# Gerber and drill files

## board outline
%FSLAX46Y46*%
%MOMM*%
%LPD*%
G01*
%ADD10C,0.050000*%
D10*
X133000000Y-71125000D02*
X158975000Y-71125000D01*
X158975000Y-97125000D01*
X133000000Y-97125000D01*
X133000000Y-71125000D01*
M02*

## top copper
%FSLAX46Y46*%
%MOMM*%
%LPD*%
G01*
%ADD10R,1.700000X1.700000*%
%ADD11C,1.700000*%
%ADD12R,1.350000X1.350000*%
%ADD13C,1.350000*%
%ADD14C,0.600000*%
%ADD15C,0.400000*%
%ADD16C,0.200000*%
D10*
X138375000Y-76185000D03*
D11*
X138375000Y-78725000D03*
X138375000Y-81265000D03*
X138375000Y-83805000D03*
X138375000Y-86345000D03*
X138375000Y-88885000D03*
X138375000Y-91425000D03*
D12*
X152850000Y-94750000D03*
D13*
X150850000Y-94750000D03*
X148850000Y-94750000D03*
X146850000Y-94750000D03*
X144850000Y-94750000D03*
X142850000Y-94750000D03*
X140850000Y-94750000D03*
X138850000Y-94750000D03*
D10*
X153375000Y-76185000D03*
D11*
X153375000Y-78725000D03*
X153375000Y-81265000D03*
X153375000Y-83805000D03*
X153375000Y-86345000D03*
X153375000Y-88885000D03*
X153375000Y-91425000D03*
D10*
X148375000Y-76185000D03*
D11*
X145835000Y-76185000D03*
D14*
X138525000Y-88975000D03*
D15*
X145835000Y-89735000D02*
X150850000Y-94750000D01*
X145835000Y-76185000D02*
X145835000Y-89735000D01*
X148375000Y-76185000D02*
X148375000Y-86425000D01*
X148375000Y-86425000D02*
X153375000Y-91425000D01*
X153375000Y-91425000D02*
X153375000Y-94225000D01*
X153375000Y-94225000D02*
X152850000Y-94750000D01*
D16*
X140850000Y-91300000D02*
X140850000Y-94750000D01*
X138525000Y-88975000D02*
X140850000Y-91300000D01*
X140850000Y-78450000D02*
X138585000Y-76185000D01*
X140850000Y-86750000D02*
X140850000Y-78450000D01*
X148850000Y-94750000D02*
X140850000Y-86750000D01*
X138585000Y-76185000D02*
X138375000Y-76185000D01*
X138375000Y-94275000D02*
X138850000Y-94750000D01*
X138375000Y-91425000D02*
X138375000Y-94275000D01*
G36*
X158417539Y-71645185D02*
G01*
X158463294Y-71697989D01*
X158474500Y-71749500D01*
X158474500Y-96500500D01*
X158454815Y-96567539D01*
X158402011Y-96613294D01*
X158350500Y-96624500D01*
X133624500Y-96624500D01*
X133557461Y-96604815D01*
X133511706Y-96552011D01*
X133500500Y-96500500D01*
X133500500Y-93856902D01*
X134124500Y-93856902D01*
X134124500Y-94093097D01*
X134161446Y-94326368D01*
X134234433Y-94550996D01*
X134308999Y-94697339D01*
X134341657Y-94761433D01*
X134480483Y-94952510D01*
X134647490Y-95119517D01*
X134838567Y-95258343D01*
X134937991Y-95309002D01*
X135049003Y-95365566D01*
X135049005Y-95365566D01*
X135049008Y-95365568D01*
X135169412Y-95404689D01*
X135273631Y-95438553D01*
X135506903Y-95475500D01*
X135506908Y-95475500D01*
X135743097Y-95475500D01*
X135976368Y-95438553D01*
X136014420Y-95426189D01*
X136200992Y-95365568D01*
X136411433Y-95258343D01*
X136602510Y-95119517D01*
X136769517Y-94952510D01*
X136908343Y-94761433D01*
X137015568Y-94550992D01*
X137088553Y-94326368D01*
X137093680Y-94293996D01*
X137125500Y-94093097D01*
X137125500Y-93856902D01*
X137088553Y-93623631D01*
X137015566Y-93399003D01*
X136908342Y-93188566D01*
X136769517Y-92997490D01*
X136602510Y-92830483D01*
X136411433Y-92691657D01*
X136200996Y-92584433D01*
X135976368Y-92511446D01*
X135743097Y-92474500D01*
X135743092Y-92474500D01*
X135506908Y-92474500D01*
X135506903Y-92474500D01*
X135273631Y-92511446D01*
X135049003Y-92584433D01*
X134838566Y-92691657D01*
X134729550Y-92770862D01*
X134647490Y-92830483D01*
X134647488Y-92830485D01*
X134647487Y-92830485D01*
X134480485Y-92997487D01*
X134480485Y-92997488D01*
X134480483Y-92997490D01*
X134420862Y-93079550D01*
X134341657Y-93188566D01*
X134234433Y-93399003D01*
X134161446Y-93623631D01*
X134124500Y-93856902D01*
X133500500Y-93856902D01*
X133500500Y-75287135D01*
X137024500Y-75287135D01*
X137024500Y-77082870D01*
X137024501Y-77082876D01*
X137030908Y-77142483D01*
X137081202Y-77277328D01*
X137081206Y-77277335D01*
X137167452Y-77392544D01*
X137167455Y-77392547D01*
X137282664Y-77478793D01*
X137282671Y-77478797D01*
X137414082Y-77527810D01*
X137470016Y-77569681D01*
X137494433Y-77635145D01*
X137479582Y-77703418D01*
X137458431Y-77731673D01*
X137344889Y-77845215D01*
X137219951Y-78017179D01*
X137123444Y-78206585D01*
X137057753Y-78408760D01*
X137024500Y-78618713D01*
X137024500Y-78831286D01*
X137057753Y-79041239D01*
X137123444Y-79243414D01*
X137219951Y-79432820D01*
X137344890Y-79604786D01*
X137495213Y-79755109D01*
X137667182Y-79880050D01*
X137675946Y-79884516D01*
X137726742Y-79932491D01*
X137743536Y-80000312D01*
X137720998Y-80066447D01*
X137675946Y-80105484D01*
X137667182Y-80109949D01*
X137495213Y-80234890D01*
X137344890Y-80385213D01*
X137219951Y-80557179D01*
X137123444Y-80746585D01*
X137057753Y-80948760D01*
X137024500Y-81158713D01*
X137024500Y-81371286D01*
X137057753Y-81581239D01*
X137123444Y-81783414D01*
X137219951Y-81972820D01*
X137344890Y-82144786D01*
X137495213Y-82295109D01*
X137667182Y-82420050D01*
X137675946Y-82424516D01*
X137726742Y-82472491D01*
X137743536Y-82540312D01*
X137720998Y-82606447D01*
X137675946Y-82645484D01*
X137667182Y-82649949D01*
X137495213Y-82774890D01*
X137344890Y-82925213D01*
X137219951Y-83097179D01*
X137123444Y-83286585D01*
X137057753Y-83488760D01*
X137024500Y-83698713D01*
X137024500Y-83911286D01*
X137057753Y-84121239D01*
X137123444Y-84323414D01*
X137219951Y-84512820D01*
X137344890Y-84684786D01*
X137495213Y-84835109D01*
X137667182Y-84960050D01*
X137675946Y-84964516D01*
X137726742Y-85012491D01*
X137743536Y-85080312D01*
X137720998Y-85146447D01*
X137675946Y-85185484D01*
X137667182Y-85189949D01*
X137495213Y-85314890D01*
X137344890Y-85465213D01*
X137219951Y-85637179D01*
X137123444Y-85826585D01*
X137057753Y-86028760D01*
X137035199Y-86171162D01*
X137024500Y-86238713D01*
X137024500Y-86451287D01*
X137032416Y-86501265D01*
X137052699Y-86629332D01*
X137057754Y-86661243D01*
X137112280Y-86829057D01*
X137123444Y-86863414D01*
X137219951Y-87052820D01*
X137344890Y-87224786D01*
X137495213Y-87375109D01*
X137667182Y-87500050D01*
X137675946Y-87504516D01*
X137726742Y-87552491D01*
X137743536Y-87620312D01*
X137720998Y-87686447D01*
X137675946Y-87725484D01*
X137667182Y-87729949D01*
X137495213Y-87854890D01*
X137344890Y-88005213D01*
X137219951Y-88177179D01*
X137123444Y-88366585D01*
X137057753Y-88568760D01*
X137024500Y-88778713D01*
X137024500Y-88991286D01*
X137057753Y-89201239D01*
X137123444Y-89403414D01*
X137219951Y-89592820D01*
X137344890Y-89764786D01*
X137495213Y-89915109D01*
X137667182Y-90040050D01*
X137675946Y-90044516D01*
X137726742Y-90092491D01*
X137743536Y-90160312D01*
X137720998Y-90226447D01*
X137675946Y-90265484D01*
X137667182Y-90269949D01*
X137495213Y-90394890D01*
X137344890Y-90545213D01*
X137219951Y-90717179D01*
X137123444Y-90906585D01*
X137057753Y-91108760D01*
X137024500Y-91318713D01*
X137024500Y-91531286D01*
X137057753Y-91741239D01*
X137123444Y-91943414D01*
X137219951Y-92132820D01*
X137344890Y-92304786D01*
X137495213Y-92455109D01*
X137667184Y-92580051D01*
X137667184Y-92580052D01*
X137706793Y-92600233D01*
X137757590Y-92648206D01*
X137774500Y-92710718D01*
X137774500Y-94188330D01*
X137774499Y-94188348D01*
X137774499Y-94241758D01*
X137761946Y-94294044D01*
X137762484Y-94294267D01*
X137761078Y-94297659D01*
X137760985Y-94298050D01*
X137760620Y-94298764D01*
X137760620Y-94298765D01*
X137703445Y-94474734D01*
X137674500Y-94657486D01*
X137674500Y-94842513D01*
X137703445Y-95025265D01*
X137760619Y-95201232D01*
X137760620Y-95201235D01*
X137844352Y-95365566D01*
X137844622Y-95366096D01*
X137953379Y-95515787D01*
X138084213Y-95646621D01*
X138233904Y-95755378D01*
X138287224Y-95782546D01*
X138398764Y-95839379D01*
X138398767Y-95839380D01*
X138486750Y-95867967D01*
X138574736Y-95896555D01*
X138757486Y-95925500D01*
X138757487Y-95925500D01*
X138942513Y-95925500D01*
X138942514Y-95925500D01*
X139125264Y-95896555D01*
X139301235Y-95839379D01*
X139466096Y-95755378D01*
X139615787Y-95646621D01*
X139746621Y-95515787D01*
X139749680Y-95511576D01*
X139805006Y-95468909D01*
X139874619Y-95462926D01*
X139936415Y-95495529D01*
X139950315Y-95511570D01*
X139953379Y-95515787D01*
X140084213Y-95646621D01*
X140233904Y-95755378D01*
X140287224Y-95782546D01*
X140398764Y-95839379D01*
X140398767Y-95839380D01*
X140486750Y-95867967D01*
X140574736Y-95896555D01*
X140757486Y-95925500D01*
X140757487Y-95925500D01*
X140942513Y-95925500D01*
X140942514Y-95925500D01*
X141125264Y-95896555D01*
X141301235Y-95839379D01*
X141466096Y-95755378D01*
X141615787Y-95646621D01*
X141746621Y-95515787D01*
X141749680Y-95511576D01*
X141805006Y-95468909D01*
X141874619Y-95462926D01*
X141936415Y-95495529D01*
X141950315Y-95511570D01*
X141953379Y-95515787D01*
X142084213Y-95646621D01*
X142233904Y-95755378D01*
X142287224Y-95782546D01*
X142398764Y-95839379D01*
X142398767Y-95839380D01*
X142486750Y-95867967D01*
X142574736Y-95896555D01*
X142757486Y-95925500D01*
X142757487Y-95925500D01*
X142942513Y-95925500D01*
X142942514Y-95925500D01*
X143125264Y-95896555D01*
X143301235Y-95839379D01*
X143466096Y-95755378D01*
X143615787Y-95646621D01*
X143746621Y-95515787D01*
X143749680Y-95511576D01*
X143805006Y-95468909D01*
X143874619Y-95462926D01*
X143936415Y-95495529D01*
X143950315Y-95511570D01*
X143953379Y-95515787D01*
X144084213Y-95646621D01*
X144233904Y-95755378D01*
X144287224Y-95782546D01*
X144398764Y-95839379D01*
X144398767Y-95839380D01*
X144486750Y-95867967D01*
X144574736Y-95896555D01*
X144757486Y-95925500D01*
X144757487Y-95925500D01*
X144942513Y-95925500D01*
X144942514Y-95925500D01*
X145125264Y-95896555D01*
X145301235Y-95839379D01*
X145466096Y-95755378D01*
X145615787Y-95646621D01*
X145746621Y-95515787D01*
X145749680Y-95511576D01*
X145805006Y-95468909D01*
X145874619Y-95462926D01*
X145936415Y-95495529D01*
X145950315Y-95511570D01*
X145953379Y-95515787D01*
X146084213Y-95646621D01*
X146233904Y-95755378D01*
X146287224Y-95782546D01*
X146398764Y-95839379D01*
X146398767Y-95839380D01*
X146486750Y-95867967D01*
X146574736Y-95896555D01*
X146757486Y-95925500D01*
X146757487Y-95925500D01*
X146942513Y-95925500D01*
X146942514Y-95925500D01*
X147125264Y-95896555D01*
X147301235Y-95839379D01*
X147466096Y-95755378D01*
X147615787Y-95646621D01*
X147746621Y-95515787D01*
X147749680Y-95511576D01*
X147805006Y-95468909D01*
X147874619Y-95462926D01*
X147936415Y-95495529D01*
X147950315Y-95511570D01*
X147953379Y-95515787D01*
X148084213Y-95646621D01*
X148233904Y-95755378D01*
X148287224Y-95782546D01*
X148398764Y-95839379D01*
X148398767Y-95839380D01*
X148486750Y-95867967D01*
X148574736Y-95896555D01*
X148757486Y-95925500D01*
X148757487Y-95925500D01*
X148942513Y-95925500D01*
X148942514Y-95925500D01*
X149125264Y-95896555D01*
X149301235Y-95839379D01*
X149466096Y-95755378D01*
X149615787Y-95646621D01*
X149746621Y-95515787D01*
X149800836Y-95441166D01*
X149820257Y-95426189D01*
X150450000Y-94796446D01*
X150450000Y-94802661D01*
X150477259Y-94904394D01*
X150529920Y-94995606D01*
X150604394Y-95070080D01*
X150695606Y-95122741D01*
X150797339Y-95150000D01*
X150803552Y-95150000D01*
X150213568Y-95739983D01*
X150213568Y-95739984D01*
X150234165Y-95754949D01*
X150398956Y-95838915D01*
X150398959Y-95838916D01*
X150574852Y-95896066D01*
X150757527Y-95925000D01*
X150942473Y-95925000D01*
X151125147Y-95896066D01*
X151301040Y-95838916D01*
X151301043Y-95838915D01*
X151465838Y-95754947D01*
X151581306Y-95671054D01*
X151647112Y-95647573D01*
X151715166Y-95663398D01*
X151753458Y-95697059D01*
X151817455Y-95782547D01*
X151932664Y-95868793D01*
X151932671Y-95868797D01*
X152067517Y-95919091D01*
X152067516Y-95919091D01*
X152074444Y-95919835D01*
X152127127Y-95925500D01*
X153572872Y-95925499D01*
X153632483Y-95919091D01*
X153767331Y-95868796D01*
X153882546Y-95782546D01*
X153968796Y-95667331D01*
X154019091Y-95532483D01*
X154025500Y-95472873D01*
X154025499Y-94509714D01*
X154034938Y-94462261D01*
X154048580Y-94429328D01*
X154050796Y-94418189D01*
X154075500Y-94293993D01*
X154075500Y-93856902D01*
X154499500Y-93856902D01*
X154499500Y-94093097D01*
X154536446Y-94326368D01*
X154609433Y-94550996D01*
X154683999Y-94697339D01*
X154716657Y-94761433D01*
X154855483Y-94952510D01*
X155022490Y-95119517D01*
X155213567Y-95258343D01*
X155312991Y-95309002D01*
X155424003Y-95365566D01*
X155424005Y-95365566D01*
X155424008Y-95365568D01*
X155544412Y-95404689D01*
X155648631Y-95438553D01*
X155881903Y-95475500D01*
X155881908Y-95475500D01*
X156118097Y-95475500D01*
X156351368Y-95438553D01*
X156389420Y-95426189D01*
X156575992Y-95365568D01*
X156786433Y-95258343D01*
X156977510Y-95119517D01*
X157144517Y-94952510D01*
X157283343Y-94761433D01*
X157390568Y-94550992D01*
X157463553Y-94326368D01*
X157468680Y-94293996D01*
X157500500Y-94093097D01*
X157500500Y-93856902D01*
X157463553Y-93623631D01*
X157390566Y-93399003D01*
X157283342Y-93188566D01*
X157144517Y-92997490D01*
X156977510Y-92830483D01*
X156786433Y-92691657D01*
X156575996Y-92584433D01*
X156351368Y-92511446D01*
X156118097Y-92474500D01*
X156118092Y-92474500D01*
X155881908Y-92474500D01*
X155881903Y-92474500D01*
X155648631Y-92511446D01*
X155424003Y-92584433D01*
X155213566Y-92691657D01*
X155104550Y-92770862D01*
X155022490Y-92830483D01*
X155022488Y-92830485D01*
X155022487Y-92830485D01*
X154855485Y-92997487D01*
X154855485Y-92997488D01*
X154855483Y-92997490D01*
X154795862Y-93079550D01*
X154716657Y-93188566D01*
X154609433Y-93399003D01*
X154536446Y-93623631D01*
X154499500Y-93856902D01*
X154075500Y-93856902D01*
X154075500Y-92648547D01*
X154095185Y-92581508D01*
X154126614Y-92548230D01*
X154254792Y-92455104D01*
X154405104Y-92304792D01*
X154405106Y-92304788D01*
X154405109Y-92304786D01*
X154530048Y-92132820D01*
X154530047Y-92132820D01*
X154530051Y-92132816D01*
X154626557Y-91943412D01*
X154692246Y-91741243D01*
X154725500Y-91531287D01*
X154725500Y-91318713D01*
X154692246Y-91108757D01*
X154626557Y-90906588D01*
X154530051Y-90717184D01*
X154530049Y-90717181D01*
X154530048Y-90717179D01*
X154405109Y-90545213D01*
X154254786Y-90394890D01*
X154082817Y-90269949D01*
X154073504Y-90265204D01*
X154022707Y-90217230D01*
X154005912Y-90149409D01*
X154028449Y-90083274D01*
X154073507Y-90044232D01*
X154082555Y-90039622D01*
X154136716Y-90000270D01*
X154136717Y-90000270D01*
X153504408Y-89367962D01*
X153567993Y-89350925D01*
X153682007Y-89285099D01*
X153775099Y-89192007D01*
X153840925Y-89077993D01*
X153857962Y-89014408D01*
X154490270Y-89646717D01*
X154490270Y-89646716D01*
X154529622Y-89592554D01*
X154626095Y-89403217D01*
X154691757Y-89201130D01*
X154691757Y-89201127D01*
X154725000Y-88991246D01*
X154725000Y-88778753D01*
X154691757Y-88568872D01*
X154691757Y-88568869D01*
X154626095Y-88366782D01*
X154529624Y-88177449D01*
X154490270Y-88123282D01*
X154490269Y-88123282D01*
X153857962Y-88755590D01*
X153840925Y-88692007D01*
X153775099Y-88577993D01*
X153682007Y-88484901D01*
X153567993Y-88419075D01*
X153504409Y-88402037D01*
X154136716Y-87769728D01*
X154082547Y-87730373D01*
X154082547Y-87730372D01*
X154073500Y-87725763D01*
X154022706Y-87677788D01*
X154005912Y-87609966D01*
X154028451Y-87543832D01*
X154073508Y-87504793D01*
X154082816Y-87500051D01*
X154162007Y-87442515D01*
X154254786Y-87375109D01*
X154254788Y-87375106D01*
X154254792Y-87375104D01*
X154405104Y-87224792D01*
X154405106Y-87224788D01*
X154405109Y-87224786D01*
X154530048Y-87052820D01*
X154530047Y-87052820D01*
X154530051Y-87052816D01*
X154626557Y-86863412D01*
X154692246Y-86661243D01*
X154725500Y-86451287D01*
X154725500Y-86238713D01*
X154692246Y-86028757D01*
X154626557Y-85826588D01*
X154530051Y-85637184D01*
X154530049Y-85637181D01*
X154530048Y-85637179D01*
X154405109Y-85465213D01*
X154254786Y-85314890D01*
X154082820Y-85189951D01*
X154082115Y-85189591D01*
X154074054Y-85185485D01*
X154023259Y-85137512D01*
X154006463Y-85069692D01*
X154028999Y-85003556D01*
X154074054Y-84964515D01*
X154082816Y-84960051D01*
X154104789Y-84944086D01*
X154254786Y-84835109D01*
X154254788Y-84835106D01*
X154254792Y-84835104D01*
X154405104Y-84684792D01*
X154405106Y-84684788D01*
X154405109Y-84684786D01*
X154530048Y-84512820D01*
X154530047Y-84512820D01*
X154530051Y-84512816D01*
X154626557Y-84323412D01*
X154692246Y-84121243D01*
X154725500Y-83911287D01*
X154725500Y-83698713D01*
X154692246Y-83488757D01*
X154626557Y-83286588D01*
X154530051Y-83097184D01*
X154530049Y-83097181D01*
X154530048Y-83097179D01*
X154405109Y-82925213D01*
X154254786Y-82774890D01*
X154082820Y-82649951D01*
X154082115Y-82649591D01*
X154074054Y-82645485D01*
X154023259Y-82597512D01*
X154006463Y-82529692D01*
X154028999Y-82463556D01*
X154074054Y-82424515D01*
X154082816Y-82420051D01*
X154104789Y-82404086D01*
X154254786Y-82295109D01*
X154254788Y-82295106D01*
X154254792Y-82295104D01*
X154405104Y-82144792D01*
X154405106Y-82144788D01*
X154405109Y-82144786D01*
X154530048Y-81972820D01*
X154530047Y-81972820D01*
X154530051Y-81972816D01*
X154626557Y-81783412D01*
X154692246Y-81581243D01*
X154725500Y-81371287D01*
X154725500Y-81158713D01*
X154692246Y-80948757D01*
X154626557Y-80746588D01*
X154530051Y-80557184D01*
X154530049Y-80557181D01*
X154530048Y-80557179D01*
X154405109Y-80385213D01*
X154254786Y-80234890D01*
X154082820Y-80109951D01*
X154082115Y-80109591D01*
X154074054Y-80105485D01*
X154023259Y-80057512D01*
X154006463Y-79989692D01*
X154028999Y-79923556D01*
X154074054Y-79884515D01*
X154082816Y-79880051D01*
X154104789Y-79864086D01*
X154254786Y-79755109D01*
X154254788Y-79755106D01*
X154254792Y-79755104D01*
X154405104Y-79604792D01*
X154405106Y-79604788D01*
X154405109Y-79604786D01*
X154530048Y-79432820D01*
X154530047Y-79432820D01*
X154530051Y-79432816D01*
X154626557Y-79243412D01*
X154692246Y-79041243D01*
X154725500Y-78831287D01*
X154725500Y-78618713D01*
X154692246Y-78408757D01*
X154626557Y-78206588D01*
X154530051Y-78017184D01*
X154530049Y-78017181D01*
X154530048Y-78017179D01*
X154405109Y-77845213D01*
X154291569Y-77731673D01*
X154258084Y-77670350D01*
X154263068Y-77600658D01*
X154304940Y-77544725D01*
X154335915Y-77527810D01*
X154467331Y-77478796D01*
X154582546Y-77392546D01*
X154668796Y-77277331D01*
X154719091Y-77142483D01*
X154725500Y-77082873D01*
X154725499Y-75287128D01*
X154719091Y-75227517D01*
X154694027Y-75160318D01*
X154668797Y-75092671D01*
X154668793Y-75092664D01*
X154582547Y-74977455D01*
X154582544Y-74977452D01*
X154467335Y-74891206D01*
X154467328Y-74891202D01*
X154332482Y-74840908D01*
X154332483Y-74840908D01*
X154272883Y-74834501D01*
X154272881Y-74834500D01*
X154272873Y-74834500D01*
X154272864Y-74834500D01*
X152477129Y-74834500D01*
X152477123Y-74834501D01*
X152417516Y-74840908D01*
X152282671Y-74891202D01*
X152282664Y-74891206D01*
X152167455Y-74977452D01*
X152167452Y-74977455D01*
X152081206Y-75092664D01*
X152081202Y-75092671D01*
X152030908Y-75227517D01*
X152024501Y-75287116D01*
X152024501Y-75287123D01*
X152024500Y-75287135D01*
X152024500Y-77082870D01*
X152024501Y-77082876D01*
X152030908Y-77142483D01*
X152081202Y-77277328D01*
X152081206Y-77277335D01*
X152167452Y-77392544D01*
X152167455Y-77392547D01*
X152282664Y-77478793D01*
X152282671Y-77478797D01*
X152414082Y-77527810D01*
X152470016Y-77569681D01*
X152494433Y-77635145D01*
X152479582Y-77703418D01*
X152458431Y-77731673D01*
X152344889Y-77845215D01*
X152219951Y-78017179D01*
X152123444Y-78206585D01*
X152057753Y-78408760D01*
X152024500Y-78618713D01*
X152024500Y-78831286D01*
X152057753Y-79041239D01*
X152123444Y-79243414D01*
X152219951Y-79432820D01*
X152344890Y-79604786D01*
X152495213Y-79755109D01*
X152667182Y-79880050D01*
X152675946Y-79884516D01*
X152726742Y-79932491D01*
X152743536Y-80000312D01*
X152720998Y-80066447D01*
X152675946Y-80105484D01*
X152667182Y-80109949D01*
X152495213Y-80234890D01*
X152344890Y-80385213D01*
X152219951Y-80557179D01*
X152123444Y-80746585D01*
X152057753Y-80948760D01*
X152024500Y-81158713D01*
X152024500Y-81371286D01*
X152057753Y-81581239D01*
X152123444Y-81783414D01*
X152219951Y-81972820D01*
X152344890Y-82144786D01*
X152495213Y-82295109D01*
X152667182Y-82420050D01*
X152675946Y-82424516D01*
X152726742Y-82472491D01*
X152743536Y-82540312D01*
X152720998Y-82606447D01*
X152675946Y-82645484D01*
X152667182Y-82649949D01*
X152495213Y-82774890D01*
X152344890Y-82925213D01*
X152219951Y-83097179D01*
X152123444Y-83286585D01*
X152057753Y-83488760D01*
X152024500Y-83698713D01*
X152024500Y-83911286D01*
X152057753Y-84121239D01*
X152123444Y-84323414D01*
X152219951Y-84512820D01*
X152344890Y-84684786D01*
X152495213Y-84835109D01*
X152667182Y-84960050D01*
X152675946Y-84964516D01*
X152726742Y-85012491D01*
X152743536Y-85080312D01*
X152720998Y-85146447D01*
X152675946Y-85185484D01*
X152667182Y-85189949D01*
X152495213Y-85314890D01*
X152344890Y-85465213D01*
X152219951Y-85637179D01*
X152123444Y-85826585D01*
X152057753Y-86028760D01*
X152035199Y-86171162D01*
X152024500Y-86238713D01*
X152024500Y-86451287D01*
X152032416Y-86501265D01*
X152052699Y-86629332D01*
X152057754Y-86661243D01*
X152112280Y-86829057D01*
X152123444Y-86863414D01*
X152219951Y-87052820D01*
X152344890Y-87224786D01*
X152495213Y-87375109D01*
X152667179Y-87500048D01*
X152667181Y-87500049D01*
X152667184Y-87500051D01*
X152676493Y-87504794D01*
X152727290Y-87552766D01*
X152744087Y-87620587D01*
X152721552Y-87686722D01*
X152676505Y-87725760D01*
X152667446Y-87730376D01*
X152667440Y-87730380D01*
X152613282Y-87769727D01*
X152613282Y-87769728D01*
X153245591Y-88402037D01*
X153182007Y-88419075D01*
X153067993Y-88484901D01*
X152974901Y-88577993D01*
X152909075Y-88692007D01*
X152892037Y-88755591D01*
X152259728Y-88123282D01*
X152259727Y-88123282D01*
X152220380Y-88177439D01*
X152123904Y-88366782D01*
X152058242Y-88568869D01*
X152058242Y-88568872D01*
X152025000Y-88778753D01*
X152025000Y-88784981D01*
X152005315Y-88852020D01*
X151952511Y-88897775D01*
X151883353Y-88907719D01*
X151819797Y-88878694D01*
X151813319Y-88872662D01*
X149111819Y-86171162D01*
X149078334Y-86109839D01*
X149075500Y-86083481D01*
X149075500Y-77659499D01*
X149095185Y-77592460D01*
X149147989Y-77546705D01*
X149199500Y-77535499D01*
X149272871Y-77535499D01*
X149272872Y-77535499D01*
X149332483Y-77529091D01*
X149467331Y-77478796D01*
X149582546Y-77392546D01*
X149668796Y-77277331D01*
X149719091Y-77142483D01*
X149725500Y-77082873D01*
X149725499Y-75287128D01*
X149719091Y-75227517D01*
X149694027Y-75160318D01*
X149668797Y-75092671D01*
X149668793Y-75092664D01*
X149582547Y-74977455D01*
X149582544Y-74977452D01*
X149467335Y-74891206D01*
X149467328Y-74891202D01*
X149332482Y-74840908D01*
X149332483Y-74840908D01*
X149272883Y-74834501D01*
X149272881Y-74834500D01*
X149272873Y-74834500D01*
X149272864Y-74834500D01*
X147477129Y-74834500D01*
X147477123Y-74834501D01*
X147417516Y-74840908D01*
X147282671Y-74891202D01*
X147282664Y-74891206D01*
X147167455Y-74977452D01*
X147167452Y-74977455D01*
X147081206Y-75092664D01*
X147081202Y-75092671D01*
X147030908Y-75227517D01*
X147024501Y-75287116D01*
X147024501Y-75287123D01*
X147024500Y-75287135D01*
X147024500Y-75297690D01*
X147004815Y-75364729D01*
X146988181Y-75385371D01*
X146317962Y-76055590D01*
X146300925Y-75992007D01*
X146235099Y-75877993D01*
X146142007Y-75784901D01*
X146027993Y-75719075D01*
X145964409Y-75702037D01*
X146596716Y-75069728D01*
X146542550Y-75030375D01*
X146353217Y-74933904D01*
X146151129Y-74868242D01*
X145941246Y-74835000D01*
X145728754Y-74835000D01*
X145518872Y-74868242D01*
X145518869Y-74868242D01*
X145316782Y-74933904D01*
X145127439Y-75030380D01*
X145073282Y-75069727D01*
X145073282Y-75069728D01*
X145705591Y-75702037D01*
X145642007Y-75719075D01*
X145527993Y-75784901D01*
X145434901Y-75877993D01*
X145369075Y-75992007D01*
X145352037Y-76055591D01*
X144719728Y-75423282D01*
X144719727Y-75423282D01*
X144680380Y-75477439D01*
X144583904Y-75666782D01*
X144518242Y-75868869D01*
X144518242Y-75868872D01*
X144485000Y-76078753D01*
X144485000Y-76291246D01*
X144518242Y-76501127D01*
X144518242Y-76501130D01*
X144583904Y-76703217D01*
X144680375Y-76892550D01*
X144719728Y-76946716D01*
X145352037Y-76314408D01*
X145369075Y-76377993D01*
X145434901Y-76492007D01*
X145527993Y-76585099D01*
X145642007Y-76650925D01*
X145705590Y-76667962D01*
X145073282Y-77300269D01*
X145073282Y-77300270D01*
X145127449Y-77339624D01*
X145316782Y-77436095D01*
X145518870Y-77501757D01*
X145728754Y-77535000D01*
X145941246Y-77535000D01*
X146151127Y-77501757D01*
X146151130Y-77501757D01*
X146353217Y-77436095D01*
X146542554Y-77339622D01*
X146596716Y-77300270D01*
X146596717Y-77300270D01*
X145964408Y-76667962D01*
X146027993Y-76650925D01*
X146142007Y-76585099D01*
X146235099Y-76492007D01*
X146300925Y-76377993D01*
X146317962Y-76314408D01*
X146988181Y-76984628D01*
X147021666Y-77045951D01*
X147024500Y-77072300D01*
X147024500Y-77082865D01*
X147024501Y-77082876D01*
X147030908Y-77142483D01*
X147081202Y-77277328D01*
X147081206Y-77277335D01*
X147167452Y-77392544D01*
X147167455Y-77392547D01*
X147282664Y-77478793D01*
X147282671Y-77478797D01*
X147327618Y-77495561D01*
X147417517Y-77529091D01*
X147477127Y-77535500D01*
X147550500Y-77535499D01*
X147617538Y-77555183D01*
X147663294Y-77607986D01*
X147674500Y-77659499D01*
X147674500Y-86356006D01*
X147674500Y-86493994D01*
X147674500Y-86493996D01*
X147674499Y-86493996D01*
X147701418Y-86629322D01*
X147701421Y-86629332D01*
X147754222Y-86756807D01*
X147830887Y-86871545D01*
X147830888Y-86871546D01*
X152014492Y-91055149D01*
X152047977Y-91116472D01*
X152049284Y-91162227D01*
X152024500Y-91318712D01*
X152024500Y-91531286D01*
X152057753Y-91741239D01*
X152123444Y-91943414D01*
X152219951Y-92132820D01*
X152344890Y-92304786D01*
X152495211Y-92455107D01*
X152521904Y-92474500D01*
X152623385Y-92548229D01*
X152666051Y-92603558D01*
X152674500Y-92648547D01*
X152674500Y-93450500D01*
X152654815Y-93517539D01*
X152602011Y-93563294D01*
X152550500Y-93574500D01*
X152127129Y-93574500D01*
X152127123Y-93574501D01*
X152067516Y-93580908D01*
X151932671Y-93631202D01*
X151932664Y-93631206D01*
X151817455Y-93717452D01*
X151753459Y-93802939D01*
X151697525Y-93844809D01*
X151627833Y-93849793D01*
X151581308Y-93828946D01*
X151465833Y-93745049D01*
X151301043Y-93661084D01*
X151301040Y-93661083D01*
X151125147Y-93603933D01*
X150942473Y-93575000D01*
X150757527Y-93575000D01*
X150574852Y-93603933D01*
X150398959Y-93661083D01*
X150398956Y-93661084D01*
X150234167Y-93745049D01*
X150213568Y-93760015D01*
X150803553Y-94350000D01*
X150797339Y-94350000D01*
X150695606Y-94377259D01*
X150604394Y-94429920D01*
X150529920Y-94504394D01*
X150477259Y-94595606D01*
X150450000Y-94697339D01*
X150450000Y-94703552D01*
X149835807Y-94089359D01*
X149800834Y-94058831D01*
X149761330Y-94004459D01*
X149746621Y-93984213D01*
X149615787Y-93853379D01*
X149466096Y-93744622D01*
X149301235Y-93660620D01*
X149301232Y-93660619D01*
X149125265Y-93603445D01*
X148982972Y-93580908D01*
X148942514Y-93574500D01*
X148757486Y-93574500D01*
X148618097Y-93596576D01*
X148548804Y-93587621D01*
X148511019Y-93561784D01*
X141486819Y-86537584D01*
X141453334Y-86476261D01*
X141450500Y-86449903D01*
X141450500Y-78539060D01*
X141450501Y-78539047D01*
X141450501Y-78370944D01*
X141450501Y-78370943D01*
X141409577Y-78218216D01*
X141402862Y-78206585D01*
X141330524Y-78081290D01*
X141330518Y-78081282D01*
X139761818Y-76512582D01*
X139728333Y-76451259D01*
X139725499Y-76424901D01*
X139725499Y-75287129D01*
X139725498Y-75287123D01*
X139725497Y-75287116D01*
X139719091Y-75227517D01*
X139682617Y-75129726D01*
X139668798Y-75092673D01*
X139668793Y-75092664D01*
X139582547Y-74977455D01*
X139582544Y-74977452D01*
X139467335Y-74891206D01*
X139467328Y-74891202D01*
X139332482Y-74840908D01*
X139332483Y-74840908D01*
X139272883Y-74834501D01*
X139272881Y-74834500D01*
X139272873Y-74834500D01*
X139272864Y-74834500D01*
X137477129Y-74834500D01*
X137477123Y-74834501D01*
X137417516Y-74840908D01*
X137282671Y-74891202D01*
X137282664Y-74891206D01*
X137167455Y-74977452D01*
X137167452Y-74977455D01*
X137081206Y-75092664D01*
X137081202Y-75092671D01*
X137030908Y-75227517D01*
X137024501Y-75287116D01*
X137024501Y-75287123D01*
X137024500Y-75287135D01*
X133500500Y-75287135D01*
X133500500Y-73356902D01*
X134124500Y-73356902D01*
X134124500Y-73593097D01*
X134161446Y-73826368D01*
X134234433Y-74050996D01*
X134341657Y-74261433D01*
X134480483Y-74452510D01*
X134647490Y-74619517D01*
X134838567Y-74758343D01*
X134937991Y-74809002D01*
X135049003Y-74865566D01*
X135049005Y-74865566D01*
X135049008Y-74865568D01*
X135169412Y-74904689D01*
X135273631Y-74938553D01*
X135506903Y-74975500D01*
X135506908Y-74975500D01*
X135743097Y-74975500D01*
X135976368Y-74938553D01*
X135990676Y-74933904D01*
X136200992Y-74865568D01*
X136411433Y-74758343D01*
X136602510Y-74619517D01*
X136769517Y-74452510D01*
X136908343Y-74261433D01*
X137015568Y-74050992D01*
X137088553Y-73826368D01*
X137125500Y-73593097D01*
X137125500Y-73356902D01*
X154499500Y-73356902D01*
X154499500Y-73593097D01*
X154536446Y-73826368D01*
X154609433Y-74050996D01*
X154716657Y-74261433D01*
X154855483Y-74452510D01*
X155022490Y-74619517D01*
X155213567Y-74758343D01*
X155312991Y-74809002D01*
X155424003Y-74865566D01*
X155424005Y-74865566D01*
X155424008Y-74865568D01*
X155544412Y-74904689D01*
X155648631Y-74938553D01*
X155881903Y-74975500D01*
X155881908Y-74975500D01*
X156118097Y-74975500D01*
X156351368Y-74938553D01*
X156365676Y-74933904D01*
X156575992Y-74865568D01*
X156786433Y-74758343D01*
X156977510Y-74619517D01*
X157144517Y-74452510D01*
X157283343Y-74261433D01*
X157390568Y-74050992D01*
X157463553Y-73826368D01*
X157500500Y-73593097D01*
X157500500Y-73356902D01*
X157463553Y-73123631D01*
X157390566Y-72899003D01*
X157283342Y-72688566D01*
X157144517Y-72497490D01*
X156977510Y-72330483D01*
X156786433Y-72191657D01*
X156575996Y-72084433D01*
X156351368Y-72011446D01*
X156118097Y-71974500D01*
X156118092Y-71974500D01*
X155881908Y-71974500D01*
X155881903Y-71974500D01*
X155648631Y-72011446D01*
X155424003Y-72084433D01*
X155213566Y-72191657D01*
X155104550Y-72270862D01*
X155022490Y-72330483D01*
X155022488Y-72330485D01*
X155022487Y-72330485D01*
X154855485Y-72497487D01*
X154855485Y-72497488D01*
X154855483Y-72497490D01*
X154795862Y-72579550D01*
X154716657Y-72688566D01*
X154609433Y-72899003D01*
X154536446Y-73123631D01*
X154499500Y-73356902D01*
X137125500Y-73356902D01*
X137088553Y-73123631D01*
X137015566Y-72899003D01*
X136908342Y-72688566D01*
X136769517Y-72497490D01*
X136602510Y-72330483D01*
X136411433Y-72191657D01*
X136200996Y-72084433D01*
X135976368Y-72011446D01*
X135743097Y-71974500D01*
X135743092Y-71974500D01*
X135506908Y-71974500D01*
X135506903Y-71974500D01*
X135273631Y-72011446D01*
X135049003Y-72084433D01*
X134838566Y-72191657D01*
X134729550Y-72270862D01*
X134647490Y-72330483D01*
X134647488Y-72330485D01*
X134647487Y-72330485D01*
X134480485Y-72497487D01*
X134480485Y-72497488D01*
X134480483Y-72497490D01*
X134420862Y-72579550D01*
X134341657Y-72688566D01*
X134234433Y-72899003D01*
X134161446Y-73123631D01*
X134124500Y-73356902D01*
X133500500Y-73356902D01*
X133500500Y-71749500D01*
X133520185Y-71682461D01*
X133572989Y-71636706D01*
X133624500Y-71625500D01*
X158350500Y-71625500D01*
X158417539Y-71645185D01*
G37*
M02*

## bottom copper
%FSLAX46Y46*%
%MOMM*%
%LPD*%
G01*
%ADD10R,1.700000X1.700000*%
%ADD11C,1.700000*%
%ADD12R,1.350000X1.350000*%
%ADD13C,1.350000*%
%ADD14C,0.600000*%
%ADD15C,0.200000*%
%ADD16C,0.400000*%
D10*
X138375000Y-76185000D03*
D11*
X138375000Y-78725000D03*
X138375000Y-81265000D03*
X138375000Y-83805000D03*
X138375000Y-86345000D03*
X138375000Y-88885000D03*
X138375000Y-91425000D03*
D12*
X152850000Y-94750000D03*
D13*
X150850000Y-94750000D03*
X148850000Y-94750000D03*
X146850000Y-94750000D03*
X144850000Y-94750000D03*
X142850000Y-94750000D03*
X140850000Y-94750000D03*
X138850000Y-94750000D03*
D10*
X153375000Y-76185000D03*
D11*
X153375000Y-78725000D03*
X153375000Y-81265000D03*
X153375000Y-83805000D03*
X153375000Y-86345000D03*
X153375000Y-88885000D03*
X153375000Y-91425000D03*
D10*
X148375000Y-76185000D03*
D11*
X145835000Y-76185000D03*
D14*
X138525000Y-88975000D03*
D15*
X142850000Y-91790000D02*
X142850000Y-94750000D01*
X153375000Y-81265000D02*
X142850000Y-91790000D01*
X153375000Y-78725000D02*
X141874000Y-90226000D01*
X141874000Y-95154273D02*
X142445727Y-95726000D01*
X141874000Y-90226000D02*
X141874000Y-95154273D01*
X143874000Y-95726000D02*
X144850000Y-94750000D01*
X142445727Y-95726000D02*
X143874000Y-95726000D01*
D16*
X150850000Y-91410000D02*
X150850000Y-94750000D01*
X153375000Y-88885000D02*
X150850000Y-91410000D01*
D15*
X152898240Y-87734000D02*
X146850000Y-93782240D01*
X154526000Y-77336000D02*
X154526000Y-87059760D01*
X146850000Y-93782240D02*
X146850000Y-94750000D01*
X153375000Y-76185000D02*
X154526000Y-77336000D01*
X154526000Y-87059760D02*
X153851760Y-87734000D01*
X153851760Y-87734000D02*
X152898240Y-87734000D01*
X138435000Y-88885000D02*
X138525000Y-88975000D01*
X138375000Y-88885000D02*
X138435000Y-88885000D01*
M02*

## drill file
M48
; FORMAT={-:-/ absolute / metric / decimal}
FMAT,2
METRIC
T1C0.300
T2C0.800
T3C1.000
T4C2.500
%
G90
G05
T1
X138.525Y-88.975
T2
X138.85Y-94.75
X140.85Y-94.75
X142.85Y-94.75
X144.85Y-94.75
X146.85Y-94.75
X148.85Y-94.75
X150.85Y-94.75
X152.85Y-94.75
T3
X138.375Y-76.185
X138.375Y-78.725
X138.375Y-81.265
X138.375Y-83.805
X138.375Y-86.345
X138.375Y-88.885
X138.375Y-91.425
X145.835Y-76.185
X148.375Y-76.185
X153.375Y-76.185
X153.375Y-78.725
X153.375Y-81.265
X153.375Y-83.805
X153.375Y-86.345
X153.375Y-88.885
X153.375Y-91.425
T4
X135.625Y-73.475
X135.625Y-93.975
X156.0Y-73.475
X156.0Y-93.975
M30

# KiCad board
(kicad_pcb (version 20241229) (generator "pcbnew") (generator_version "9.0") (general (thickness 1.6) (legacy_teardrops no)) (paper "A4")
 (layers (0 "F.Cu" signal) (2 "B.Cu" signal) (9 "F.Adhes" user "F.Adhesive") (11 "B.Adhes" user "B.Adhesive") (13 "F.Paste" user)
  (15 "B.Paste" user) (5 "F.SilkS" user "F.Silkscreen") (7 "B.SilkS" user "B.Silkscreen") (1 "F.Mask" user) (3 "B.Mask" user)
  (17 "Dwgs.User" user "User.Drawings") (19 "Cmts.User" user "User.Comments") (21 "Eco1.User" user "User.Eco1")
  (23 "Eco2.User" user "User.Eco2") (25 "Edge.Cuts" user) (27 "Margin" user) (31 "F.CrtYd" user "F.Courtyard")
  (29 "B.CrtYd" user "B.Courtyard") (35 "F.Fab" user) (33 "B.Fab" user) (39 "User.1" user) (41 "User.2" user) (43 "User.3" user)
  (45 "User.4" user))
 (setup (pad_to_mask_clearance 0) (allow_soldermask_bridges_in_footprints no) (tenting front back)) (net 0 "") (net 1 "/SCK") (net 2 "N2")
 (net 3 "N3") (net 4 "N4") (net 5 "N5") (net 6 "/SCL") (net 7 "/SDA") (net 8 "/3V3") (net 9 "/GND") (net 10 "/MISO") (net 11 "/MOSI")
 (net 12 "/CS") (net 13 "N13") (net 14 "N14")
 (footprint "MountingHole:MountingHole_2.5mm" (layer "F.Cu") (at 135.625 73.475)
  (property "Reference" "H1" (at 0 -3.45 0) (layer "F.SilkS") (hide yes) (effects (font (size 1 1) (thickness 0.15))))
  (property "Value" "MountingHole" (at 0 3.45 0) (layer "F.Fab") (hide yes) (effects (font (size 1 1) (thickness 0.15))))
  (pad "" np_thru_hole circle (at 0 0) (size 2.5 2.5) (drill 2.5) (layers "*.Cu" "*.Mask")))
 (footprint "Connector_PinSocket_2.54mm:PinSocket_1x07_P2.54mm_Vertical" (layer "F.Cu") (at 138.375 76.185)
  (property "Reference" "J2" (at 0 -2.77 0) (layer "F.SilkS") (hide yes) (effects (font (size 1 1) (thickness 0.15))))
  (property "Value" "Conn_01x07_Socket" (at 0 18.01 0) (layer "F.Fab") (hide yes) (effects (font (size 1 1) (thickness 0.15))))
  (pad "1" thru_hole rect (at 0 0) (size 1.7 1.7) (drill 1) (layers "*.Cu" "*.Mask") (remove_unused_layers no) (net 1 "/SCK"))
  (pad "2" thru_hole circle (at 0 2.54) (size 1.7 1.7) (drill 1) (layers "*.Cu" "*.Mask") (remove_unused_layers no) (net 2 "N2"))
  (pad "3" thru_hole circle (at 0 5.08) (size 1.7 1.7) (drill 1) (layers "*.Cu" "*.Mask") (remove_unused_layers no) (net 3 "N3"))
  (pad "4" thru_hole circle (at 0 7.62) (size 1.7 1.7) (drill 1) (layers "*.Cu" "*.Mask") (remove_unused_layers no) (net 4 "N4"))
  (pad "5" thru_hole circle (at 0 10.16) (size 1.7 1.7) (drill 1) (layers "*.Cu" "*.Mask") (remove_unused_layers no) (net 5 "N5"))
  (pad "6" thru_hole circle (at 0 12.7) (size 1.7 1.7) (drill 1) (layers "*.Cu" "*.Mask") (remove_unused_layers no) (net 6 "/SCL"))
  (pad "7" thru_hole circle (at 0 15.24) (size 1.7 1.7) (drill 1) (layers "*.Cu" "*.Mask") (remove_unused_layers no) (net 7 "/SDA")))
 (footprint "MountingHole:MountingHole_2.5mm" (layer "F.Cu") (at 156.125 93.975)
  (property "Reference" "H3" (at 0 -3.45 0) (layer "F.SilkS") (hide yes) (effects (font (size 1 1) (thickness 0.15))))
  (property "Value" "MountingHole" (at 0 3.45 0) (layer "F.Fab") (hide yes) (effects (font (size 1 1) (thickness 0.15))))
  (pad "" np_thru_hole circle (at -0.125 0) (size 2.5 2.5) (drill 2.5) (layers "*.Cu" "*.Mask")))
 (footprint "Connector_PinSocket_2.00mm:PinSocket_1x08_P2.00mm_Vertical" (layer "F.Cu") (at 152.85 94.75 -90)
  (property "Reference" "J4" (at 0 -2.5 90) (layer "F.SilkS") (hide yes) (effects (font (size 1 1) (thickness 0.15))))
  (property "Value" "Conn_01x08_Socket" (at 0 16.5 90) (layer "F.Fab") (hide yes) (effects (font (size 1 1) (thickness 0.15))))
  (pad "1" thru_hole rect (at 0 0 270) (size 1.35 1.35) (drill 0.8) (layers "*.Cu" "*.Mask") (remove_unused_layers no) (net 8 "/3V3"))
  (pad "2" thru_hole circle (at 0 2 270) (size 1.35 1.35) (drill 0.8) (layers "*.Cu" "*.Mask") (remove_unused_layers no) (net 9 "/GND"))
  (pad "3" thru_hole circle (at 0 4 270) (size 1.35 1.35) (drill 0.8) (layers "*.Cu" "*.Mask") (remove_unused_layers no) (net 1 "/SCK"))
  (pad "4" thru_hole circle (at 0 6 270) (size 1.35 1.35) (drill 0.8) (layers "*.Cu" "*.Mask") (remove_unused_layers no) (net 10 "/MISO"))
  (pad "5" thru_hole circle (at 0 8 270) (size 1.35 1.35) (drill 0.8) (layers "*.Cu" "*.Mask") (remove_unused_layers no) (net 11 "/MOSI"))
  (pad "6" thru_hole circle (at 0 10 270) (size 1.35 1.35) (drill 0.8) (layers "*.Cu" "*.Mask") (remove_unused_layers no) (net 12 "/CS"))
  (pad "7" thru_hole circle (at 0 12 270) (size 1.35 1.35) (drill 0.8) (layers "*.Cu" "*.Mask") (remove_unused_layers no) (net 6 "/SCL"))
  (pad "8" thru_hole circle (at 0 14 270) (size 1.35 1.35) (drill 0.8) (layers "*.Cu" "*.Mask") (remove_unused_layers no) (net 7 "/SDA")))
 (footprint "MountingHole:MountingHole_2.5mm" (layer "F.Cu") (at 156.125 73.475)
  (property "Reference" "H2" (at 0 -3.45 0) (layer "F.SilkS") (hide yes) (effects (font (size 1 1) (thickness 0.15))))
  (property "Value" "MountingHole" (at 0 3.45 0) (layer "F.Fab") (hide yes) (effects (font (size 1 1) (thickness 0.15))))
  (pad "" np_thru_hole circle (at -0.125 0) (size 2.5 2.5) (drill 2.5) (layers "*.Cu" "*.Mask")))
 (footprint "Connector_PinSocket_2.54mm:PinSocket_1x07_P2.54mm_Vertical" (layer "F.Cu") (at 153.375 76.185)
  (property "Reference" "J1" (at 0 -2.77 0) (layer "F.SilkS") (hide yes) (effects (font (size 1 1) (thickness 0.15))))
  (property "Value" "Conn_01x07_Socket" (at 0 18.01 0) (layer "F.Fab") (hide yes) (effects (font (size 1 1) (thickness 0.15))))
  (pad "1" thru_hole rect (at 0 0) (size 1.7 1.7) (drill 1) (layers "*.Cu" "*.Mask") (remove_unused_layers no) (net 10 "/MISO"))
  (pad "2" thru_hole circle (at 0 2.54) (size 1.7 1.7) (drill 1) (layers "*.Cu" "*.Mask") (remove_unused_layers no) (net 11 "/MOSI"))
  (pad "3" thru_hole circle (at 0 5.08) (size 1.7 1.7) (drill 1) (layers "*.Cu" "*.Mask") (remove_unused_layers no) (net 12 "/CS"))
  (pad "4" thru_hole circle (at 0 7.62) (size 1.7 1.7) (drill 1) (layers "*.Cu" "*.Mask") (remove_unused_layers no) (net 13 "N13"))
  (pad "5" thru_hole circle (at 0 10.16) (size 1.7 1.7) (drill 1) (layers "*.Cu" "*.Mask") (remove_unused_layers no) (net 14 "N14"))
  (pad "6" thru_hole circle (at 0 12.7) (size 1.7 1.7) (drill 1) (layers "*.Cu" "*.Mask") (remove_unused_layers no) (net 9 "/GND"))
  (pad "7" thru_hole circle (at 0 15.24) (size 1.7 1.7) (drill 1) (layers "*.Cu" "*.Mask") (remove_unused_layers no) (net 8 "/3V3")))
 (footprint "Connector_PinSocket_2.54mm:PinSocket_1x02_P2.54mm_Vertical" (layer "F.Cu") (at 148.375 76.185 -90)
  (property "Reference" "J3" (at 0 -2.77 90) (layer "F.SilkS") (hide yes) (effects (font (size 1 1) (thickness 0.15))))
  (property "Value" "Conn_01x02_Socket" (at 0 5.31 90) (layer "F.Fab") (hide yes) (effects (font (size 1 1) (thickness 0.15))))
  (pad "1" thru_hole rect (at 0 0 270) (size 1.7 1.7) (drill 1) (layers "*.Cu" "*.Mask") (remove_unused_layers no) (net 8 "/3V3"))
  (pad "2" thru_hole circle (at 0 2.54 270) (size 1.7 1.7) (drill 1) (layers "*.Cu" "*.Mask") (remove_unused_layers no) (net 9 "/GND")))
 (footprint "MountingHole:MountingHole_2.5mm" (layer "F.Cu") (at 135.625 93.975)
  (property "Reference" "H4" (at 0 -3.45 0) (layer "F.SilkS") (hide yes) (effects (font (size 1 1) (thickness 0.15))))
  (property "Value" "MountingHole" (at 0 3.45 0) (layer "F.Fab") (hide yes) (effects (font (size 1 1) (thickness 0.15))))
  (pad "" np_thru_hole circle (at 0 0) (size 2.5 2.5) (drill 2.5) (layers "*.Cu" "*.Mask")))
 (gr_rect (start 133 71.125) (end 158.975 97.125) (stroke (width 0.05) (type default)) (fill no) (layer "Edge.Cuts"))
 (segment (start 142.85 91.79) (end 142.85 94.75) (width 0.2) (layer "B.Cu") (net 12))
 (segment (start 153.375 81.265) (end 142.85 91.79) (width 0.2) (layer "B.Cu") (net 12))
 (segment (start 153.375 78.725) (end 141.874 90.226) (width 0.2) (layer "B.Cu") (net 11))
 (segment (start 141.874 95.154273) (end 142.445727 95.726) (width 0.2) (layer "B.Cu") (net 11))
 (segment (start 141.874 90.226) (end 141.874 95.154273) (width 0.2) (layer "B.Cu") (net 11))
 (segment (start 143.874 95.726) (end 144.85 94.75) (width 0.2) (layer "B.Cu") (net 11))
 (segment (start 142.445727 95.726) (end 143.874 95.726) (width 0.2) (layer "B.Cu") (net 11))
 (segment (start 145.835 89.735) (end 150.85 94.75) (width 0.4) (layer "F.Cu") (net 9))
 (segment (start 145.835 76.185) (end 145.835 89.735) (width 0.4) (layer "F.Cu") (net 9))
 (segment (start 150.85 91.41) (end 150.85 94.75) (width 0.4) (layer "B.Cu") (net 9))
 (segment (start 153.375 88.885) (end 150.85 91.41) (width 0.4) (layer "B.Cu") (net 9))
 (segment (start 152.89824 87.734) (end 146.85 93.78224) (width 0.2) (layer "B.Cu") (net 10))
 (segment (start 154.526 77.336) (end 154.526 87.05976) (width 0.2) (layer "B.Cu") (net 10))
 (segment (start 146.85 93.78224) (end 146.85 94.75) (width 0.2) (layer "B.Cu") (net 10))
 (segment (start 153.375 76.185) (end 154.526 77.336) (width 0.2) (layer "B.Cu") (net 10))
 (segment (start 154.526 87.05976) (end 153.85176 87.734) (width 0.2) (layer "B.Cu") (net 10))
 (segment (start 153.85176 87.734) (end 152.89824 87.734) (width 0.2) (layer "B.Cu") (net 10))
 (segment (start 148.375 76.185) (end 148.375 86.425) (width 0.4) (layer "F.Cu") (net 8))
 (segment (start 148.375 86.425) (end 153.375 91.425) (width 0.4) (layer "F.Cu") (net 8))
 (segment (start 153.375 91.425) (end 153.375 94.225) (width 0.4) (layer "F.Cu") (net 8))
 (segment (start 153.375 94.225) (end 152.85 94.75) (width 0.4) (layer "F.Cu") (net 8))
 (segment (start 140.85 91.3) (end 140.85 94.75) (width 0.2) (layer "F.Cu") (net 6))
 (segment (start 138.525 88.975) (end 140.85 91.3) (width 0.2) (layer "F.Cu") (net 6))
 (via (at 138.525 88.975) (size 0.6) (drill 0.3) (layers "F.Cu" "B.Cu") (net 6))
 (segment (start 138.435 88.885) (end 138.525 88.975) (width 0.2) (layer "B.Cu") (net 6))
 (segment (start 138.375 88.885) (end 138.435 88.885) (width 0.2) (layer "B.Cu") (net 6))
 (segment (start 140.85 78.45) (end 138.585 76.185) (width 0.2) (layer "F.Cu") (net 1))
 (segment (start 140.85 86.75) (end 140.85 78.45) (width 0.2) (layer "F.Cu") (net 1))
 (segment (start 148.85 94.75) (end 140.85 86.75) (width 0.2) (layer "F.Cu") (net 1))
 (segment (start 138.585 76.185) (end 138.375 76.185) (width 0.2) (layer "F.Cu") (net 1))
 (segment (start 138.375 94.275) (end 138.85 94.75) (width 0.2) (layer "F.Cu") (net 7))
 (segment (start 138.375 91.425) (end 138.375 94.275) (width 0.2) (layer "F.Cu") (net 7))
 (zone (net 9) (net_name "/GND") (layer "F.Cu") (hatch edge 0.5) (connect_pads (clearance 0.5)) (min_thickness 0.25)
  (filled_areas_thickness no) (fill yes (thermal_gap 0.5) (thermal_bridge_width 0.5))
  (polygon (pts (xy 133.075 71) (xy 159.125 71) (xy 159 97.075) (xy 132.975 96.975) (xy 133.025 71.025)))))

